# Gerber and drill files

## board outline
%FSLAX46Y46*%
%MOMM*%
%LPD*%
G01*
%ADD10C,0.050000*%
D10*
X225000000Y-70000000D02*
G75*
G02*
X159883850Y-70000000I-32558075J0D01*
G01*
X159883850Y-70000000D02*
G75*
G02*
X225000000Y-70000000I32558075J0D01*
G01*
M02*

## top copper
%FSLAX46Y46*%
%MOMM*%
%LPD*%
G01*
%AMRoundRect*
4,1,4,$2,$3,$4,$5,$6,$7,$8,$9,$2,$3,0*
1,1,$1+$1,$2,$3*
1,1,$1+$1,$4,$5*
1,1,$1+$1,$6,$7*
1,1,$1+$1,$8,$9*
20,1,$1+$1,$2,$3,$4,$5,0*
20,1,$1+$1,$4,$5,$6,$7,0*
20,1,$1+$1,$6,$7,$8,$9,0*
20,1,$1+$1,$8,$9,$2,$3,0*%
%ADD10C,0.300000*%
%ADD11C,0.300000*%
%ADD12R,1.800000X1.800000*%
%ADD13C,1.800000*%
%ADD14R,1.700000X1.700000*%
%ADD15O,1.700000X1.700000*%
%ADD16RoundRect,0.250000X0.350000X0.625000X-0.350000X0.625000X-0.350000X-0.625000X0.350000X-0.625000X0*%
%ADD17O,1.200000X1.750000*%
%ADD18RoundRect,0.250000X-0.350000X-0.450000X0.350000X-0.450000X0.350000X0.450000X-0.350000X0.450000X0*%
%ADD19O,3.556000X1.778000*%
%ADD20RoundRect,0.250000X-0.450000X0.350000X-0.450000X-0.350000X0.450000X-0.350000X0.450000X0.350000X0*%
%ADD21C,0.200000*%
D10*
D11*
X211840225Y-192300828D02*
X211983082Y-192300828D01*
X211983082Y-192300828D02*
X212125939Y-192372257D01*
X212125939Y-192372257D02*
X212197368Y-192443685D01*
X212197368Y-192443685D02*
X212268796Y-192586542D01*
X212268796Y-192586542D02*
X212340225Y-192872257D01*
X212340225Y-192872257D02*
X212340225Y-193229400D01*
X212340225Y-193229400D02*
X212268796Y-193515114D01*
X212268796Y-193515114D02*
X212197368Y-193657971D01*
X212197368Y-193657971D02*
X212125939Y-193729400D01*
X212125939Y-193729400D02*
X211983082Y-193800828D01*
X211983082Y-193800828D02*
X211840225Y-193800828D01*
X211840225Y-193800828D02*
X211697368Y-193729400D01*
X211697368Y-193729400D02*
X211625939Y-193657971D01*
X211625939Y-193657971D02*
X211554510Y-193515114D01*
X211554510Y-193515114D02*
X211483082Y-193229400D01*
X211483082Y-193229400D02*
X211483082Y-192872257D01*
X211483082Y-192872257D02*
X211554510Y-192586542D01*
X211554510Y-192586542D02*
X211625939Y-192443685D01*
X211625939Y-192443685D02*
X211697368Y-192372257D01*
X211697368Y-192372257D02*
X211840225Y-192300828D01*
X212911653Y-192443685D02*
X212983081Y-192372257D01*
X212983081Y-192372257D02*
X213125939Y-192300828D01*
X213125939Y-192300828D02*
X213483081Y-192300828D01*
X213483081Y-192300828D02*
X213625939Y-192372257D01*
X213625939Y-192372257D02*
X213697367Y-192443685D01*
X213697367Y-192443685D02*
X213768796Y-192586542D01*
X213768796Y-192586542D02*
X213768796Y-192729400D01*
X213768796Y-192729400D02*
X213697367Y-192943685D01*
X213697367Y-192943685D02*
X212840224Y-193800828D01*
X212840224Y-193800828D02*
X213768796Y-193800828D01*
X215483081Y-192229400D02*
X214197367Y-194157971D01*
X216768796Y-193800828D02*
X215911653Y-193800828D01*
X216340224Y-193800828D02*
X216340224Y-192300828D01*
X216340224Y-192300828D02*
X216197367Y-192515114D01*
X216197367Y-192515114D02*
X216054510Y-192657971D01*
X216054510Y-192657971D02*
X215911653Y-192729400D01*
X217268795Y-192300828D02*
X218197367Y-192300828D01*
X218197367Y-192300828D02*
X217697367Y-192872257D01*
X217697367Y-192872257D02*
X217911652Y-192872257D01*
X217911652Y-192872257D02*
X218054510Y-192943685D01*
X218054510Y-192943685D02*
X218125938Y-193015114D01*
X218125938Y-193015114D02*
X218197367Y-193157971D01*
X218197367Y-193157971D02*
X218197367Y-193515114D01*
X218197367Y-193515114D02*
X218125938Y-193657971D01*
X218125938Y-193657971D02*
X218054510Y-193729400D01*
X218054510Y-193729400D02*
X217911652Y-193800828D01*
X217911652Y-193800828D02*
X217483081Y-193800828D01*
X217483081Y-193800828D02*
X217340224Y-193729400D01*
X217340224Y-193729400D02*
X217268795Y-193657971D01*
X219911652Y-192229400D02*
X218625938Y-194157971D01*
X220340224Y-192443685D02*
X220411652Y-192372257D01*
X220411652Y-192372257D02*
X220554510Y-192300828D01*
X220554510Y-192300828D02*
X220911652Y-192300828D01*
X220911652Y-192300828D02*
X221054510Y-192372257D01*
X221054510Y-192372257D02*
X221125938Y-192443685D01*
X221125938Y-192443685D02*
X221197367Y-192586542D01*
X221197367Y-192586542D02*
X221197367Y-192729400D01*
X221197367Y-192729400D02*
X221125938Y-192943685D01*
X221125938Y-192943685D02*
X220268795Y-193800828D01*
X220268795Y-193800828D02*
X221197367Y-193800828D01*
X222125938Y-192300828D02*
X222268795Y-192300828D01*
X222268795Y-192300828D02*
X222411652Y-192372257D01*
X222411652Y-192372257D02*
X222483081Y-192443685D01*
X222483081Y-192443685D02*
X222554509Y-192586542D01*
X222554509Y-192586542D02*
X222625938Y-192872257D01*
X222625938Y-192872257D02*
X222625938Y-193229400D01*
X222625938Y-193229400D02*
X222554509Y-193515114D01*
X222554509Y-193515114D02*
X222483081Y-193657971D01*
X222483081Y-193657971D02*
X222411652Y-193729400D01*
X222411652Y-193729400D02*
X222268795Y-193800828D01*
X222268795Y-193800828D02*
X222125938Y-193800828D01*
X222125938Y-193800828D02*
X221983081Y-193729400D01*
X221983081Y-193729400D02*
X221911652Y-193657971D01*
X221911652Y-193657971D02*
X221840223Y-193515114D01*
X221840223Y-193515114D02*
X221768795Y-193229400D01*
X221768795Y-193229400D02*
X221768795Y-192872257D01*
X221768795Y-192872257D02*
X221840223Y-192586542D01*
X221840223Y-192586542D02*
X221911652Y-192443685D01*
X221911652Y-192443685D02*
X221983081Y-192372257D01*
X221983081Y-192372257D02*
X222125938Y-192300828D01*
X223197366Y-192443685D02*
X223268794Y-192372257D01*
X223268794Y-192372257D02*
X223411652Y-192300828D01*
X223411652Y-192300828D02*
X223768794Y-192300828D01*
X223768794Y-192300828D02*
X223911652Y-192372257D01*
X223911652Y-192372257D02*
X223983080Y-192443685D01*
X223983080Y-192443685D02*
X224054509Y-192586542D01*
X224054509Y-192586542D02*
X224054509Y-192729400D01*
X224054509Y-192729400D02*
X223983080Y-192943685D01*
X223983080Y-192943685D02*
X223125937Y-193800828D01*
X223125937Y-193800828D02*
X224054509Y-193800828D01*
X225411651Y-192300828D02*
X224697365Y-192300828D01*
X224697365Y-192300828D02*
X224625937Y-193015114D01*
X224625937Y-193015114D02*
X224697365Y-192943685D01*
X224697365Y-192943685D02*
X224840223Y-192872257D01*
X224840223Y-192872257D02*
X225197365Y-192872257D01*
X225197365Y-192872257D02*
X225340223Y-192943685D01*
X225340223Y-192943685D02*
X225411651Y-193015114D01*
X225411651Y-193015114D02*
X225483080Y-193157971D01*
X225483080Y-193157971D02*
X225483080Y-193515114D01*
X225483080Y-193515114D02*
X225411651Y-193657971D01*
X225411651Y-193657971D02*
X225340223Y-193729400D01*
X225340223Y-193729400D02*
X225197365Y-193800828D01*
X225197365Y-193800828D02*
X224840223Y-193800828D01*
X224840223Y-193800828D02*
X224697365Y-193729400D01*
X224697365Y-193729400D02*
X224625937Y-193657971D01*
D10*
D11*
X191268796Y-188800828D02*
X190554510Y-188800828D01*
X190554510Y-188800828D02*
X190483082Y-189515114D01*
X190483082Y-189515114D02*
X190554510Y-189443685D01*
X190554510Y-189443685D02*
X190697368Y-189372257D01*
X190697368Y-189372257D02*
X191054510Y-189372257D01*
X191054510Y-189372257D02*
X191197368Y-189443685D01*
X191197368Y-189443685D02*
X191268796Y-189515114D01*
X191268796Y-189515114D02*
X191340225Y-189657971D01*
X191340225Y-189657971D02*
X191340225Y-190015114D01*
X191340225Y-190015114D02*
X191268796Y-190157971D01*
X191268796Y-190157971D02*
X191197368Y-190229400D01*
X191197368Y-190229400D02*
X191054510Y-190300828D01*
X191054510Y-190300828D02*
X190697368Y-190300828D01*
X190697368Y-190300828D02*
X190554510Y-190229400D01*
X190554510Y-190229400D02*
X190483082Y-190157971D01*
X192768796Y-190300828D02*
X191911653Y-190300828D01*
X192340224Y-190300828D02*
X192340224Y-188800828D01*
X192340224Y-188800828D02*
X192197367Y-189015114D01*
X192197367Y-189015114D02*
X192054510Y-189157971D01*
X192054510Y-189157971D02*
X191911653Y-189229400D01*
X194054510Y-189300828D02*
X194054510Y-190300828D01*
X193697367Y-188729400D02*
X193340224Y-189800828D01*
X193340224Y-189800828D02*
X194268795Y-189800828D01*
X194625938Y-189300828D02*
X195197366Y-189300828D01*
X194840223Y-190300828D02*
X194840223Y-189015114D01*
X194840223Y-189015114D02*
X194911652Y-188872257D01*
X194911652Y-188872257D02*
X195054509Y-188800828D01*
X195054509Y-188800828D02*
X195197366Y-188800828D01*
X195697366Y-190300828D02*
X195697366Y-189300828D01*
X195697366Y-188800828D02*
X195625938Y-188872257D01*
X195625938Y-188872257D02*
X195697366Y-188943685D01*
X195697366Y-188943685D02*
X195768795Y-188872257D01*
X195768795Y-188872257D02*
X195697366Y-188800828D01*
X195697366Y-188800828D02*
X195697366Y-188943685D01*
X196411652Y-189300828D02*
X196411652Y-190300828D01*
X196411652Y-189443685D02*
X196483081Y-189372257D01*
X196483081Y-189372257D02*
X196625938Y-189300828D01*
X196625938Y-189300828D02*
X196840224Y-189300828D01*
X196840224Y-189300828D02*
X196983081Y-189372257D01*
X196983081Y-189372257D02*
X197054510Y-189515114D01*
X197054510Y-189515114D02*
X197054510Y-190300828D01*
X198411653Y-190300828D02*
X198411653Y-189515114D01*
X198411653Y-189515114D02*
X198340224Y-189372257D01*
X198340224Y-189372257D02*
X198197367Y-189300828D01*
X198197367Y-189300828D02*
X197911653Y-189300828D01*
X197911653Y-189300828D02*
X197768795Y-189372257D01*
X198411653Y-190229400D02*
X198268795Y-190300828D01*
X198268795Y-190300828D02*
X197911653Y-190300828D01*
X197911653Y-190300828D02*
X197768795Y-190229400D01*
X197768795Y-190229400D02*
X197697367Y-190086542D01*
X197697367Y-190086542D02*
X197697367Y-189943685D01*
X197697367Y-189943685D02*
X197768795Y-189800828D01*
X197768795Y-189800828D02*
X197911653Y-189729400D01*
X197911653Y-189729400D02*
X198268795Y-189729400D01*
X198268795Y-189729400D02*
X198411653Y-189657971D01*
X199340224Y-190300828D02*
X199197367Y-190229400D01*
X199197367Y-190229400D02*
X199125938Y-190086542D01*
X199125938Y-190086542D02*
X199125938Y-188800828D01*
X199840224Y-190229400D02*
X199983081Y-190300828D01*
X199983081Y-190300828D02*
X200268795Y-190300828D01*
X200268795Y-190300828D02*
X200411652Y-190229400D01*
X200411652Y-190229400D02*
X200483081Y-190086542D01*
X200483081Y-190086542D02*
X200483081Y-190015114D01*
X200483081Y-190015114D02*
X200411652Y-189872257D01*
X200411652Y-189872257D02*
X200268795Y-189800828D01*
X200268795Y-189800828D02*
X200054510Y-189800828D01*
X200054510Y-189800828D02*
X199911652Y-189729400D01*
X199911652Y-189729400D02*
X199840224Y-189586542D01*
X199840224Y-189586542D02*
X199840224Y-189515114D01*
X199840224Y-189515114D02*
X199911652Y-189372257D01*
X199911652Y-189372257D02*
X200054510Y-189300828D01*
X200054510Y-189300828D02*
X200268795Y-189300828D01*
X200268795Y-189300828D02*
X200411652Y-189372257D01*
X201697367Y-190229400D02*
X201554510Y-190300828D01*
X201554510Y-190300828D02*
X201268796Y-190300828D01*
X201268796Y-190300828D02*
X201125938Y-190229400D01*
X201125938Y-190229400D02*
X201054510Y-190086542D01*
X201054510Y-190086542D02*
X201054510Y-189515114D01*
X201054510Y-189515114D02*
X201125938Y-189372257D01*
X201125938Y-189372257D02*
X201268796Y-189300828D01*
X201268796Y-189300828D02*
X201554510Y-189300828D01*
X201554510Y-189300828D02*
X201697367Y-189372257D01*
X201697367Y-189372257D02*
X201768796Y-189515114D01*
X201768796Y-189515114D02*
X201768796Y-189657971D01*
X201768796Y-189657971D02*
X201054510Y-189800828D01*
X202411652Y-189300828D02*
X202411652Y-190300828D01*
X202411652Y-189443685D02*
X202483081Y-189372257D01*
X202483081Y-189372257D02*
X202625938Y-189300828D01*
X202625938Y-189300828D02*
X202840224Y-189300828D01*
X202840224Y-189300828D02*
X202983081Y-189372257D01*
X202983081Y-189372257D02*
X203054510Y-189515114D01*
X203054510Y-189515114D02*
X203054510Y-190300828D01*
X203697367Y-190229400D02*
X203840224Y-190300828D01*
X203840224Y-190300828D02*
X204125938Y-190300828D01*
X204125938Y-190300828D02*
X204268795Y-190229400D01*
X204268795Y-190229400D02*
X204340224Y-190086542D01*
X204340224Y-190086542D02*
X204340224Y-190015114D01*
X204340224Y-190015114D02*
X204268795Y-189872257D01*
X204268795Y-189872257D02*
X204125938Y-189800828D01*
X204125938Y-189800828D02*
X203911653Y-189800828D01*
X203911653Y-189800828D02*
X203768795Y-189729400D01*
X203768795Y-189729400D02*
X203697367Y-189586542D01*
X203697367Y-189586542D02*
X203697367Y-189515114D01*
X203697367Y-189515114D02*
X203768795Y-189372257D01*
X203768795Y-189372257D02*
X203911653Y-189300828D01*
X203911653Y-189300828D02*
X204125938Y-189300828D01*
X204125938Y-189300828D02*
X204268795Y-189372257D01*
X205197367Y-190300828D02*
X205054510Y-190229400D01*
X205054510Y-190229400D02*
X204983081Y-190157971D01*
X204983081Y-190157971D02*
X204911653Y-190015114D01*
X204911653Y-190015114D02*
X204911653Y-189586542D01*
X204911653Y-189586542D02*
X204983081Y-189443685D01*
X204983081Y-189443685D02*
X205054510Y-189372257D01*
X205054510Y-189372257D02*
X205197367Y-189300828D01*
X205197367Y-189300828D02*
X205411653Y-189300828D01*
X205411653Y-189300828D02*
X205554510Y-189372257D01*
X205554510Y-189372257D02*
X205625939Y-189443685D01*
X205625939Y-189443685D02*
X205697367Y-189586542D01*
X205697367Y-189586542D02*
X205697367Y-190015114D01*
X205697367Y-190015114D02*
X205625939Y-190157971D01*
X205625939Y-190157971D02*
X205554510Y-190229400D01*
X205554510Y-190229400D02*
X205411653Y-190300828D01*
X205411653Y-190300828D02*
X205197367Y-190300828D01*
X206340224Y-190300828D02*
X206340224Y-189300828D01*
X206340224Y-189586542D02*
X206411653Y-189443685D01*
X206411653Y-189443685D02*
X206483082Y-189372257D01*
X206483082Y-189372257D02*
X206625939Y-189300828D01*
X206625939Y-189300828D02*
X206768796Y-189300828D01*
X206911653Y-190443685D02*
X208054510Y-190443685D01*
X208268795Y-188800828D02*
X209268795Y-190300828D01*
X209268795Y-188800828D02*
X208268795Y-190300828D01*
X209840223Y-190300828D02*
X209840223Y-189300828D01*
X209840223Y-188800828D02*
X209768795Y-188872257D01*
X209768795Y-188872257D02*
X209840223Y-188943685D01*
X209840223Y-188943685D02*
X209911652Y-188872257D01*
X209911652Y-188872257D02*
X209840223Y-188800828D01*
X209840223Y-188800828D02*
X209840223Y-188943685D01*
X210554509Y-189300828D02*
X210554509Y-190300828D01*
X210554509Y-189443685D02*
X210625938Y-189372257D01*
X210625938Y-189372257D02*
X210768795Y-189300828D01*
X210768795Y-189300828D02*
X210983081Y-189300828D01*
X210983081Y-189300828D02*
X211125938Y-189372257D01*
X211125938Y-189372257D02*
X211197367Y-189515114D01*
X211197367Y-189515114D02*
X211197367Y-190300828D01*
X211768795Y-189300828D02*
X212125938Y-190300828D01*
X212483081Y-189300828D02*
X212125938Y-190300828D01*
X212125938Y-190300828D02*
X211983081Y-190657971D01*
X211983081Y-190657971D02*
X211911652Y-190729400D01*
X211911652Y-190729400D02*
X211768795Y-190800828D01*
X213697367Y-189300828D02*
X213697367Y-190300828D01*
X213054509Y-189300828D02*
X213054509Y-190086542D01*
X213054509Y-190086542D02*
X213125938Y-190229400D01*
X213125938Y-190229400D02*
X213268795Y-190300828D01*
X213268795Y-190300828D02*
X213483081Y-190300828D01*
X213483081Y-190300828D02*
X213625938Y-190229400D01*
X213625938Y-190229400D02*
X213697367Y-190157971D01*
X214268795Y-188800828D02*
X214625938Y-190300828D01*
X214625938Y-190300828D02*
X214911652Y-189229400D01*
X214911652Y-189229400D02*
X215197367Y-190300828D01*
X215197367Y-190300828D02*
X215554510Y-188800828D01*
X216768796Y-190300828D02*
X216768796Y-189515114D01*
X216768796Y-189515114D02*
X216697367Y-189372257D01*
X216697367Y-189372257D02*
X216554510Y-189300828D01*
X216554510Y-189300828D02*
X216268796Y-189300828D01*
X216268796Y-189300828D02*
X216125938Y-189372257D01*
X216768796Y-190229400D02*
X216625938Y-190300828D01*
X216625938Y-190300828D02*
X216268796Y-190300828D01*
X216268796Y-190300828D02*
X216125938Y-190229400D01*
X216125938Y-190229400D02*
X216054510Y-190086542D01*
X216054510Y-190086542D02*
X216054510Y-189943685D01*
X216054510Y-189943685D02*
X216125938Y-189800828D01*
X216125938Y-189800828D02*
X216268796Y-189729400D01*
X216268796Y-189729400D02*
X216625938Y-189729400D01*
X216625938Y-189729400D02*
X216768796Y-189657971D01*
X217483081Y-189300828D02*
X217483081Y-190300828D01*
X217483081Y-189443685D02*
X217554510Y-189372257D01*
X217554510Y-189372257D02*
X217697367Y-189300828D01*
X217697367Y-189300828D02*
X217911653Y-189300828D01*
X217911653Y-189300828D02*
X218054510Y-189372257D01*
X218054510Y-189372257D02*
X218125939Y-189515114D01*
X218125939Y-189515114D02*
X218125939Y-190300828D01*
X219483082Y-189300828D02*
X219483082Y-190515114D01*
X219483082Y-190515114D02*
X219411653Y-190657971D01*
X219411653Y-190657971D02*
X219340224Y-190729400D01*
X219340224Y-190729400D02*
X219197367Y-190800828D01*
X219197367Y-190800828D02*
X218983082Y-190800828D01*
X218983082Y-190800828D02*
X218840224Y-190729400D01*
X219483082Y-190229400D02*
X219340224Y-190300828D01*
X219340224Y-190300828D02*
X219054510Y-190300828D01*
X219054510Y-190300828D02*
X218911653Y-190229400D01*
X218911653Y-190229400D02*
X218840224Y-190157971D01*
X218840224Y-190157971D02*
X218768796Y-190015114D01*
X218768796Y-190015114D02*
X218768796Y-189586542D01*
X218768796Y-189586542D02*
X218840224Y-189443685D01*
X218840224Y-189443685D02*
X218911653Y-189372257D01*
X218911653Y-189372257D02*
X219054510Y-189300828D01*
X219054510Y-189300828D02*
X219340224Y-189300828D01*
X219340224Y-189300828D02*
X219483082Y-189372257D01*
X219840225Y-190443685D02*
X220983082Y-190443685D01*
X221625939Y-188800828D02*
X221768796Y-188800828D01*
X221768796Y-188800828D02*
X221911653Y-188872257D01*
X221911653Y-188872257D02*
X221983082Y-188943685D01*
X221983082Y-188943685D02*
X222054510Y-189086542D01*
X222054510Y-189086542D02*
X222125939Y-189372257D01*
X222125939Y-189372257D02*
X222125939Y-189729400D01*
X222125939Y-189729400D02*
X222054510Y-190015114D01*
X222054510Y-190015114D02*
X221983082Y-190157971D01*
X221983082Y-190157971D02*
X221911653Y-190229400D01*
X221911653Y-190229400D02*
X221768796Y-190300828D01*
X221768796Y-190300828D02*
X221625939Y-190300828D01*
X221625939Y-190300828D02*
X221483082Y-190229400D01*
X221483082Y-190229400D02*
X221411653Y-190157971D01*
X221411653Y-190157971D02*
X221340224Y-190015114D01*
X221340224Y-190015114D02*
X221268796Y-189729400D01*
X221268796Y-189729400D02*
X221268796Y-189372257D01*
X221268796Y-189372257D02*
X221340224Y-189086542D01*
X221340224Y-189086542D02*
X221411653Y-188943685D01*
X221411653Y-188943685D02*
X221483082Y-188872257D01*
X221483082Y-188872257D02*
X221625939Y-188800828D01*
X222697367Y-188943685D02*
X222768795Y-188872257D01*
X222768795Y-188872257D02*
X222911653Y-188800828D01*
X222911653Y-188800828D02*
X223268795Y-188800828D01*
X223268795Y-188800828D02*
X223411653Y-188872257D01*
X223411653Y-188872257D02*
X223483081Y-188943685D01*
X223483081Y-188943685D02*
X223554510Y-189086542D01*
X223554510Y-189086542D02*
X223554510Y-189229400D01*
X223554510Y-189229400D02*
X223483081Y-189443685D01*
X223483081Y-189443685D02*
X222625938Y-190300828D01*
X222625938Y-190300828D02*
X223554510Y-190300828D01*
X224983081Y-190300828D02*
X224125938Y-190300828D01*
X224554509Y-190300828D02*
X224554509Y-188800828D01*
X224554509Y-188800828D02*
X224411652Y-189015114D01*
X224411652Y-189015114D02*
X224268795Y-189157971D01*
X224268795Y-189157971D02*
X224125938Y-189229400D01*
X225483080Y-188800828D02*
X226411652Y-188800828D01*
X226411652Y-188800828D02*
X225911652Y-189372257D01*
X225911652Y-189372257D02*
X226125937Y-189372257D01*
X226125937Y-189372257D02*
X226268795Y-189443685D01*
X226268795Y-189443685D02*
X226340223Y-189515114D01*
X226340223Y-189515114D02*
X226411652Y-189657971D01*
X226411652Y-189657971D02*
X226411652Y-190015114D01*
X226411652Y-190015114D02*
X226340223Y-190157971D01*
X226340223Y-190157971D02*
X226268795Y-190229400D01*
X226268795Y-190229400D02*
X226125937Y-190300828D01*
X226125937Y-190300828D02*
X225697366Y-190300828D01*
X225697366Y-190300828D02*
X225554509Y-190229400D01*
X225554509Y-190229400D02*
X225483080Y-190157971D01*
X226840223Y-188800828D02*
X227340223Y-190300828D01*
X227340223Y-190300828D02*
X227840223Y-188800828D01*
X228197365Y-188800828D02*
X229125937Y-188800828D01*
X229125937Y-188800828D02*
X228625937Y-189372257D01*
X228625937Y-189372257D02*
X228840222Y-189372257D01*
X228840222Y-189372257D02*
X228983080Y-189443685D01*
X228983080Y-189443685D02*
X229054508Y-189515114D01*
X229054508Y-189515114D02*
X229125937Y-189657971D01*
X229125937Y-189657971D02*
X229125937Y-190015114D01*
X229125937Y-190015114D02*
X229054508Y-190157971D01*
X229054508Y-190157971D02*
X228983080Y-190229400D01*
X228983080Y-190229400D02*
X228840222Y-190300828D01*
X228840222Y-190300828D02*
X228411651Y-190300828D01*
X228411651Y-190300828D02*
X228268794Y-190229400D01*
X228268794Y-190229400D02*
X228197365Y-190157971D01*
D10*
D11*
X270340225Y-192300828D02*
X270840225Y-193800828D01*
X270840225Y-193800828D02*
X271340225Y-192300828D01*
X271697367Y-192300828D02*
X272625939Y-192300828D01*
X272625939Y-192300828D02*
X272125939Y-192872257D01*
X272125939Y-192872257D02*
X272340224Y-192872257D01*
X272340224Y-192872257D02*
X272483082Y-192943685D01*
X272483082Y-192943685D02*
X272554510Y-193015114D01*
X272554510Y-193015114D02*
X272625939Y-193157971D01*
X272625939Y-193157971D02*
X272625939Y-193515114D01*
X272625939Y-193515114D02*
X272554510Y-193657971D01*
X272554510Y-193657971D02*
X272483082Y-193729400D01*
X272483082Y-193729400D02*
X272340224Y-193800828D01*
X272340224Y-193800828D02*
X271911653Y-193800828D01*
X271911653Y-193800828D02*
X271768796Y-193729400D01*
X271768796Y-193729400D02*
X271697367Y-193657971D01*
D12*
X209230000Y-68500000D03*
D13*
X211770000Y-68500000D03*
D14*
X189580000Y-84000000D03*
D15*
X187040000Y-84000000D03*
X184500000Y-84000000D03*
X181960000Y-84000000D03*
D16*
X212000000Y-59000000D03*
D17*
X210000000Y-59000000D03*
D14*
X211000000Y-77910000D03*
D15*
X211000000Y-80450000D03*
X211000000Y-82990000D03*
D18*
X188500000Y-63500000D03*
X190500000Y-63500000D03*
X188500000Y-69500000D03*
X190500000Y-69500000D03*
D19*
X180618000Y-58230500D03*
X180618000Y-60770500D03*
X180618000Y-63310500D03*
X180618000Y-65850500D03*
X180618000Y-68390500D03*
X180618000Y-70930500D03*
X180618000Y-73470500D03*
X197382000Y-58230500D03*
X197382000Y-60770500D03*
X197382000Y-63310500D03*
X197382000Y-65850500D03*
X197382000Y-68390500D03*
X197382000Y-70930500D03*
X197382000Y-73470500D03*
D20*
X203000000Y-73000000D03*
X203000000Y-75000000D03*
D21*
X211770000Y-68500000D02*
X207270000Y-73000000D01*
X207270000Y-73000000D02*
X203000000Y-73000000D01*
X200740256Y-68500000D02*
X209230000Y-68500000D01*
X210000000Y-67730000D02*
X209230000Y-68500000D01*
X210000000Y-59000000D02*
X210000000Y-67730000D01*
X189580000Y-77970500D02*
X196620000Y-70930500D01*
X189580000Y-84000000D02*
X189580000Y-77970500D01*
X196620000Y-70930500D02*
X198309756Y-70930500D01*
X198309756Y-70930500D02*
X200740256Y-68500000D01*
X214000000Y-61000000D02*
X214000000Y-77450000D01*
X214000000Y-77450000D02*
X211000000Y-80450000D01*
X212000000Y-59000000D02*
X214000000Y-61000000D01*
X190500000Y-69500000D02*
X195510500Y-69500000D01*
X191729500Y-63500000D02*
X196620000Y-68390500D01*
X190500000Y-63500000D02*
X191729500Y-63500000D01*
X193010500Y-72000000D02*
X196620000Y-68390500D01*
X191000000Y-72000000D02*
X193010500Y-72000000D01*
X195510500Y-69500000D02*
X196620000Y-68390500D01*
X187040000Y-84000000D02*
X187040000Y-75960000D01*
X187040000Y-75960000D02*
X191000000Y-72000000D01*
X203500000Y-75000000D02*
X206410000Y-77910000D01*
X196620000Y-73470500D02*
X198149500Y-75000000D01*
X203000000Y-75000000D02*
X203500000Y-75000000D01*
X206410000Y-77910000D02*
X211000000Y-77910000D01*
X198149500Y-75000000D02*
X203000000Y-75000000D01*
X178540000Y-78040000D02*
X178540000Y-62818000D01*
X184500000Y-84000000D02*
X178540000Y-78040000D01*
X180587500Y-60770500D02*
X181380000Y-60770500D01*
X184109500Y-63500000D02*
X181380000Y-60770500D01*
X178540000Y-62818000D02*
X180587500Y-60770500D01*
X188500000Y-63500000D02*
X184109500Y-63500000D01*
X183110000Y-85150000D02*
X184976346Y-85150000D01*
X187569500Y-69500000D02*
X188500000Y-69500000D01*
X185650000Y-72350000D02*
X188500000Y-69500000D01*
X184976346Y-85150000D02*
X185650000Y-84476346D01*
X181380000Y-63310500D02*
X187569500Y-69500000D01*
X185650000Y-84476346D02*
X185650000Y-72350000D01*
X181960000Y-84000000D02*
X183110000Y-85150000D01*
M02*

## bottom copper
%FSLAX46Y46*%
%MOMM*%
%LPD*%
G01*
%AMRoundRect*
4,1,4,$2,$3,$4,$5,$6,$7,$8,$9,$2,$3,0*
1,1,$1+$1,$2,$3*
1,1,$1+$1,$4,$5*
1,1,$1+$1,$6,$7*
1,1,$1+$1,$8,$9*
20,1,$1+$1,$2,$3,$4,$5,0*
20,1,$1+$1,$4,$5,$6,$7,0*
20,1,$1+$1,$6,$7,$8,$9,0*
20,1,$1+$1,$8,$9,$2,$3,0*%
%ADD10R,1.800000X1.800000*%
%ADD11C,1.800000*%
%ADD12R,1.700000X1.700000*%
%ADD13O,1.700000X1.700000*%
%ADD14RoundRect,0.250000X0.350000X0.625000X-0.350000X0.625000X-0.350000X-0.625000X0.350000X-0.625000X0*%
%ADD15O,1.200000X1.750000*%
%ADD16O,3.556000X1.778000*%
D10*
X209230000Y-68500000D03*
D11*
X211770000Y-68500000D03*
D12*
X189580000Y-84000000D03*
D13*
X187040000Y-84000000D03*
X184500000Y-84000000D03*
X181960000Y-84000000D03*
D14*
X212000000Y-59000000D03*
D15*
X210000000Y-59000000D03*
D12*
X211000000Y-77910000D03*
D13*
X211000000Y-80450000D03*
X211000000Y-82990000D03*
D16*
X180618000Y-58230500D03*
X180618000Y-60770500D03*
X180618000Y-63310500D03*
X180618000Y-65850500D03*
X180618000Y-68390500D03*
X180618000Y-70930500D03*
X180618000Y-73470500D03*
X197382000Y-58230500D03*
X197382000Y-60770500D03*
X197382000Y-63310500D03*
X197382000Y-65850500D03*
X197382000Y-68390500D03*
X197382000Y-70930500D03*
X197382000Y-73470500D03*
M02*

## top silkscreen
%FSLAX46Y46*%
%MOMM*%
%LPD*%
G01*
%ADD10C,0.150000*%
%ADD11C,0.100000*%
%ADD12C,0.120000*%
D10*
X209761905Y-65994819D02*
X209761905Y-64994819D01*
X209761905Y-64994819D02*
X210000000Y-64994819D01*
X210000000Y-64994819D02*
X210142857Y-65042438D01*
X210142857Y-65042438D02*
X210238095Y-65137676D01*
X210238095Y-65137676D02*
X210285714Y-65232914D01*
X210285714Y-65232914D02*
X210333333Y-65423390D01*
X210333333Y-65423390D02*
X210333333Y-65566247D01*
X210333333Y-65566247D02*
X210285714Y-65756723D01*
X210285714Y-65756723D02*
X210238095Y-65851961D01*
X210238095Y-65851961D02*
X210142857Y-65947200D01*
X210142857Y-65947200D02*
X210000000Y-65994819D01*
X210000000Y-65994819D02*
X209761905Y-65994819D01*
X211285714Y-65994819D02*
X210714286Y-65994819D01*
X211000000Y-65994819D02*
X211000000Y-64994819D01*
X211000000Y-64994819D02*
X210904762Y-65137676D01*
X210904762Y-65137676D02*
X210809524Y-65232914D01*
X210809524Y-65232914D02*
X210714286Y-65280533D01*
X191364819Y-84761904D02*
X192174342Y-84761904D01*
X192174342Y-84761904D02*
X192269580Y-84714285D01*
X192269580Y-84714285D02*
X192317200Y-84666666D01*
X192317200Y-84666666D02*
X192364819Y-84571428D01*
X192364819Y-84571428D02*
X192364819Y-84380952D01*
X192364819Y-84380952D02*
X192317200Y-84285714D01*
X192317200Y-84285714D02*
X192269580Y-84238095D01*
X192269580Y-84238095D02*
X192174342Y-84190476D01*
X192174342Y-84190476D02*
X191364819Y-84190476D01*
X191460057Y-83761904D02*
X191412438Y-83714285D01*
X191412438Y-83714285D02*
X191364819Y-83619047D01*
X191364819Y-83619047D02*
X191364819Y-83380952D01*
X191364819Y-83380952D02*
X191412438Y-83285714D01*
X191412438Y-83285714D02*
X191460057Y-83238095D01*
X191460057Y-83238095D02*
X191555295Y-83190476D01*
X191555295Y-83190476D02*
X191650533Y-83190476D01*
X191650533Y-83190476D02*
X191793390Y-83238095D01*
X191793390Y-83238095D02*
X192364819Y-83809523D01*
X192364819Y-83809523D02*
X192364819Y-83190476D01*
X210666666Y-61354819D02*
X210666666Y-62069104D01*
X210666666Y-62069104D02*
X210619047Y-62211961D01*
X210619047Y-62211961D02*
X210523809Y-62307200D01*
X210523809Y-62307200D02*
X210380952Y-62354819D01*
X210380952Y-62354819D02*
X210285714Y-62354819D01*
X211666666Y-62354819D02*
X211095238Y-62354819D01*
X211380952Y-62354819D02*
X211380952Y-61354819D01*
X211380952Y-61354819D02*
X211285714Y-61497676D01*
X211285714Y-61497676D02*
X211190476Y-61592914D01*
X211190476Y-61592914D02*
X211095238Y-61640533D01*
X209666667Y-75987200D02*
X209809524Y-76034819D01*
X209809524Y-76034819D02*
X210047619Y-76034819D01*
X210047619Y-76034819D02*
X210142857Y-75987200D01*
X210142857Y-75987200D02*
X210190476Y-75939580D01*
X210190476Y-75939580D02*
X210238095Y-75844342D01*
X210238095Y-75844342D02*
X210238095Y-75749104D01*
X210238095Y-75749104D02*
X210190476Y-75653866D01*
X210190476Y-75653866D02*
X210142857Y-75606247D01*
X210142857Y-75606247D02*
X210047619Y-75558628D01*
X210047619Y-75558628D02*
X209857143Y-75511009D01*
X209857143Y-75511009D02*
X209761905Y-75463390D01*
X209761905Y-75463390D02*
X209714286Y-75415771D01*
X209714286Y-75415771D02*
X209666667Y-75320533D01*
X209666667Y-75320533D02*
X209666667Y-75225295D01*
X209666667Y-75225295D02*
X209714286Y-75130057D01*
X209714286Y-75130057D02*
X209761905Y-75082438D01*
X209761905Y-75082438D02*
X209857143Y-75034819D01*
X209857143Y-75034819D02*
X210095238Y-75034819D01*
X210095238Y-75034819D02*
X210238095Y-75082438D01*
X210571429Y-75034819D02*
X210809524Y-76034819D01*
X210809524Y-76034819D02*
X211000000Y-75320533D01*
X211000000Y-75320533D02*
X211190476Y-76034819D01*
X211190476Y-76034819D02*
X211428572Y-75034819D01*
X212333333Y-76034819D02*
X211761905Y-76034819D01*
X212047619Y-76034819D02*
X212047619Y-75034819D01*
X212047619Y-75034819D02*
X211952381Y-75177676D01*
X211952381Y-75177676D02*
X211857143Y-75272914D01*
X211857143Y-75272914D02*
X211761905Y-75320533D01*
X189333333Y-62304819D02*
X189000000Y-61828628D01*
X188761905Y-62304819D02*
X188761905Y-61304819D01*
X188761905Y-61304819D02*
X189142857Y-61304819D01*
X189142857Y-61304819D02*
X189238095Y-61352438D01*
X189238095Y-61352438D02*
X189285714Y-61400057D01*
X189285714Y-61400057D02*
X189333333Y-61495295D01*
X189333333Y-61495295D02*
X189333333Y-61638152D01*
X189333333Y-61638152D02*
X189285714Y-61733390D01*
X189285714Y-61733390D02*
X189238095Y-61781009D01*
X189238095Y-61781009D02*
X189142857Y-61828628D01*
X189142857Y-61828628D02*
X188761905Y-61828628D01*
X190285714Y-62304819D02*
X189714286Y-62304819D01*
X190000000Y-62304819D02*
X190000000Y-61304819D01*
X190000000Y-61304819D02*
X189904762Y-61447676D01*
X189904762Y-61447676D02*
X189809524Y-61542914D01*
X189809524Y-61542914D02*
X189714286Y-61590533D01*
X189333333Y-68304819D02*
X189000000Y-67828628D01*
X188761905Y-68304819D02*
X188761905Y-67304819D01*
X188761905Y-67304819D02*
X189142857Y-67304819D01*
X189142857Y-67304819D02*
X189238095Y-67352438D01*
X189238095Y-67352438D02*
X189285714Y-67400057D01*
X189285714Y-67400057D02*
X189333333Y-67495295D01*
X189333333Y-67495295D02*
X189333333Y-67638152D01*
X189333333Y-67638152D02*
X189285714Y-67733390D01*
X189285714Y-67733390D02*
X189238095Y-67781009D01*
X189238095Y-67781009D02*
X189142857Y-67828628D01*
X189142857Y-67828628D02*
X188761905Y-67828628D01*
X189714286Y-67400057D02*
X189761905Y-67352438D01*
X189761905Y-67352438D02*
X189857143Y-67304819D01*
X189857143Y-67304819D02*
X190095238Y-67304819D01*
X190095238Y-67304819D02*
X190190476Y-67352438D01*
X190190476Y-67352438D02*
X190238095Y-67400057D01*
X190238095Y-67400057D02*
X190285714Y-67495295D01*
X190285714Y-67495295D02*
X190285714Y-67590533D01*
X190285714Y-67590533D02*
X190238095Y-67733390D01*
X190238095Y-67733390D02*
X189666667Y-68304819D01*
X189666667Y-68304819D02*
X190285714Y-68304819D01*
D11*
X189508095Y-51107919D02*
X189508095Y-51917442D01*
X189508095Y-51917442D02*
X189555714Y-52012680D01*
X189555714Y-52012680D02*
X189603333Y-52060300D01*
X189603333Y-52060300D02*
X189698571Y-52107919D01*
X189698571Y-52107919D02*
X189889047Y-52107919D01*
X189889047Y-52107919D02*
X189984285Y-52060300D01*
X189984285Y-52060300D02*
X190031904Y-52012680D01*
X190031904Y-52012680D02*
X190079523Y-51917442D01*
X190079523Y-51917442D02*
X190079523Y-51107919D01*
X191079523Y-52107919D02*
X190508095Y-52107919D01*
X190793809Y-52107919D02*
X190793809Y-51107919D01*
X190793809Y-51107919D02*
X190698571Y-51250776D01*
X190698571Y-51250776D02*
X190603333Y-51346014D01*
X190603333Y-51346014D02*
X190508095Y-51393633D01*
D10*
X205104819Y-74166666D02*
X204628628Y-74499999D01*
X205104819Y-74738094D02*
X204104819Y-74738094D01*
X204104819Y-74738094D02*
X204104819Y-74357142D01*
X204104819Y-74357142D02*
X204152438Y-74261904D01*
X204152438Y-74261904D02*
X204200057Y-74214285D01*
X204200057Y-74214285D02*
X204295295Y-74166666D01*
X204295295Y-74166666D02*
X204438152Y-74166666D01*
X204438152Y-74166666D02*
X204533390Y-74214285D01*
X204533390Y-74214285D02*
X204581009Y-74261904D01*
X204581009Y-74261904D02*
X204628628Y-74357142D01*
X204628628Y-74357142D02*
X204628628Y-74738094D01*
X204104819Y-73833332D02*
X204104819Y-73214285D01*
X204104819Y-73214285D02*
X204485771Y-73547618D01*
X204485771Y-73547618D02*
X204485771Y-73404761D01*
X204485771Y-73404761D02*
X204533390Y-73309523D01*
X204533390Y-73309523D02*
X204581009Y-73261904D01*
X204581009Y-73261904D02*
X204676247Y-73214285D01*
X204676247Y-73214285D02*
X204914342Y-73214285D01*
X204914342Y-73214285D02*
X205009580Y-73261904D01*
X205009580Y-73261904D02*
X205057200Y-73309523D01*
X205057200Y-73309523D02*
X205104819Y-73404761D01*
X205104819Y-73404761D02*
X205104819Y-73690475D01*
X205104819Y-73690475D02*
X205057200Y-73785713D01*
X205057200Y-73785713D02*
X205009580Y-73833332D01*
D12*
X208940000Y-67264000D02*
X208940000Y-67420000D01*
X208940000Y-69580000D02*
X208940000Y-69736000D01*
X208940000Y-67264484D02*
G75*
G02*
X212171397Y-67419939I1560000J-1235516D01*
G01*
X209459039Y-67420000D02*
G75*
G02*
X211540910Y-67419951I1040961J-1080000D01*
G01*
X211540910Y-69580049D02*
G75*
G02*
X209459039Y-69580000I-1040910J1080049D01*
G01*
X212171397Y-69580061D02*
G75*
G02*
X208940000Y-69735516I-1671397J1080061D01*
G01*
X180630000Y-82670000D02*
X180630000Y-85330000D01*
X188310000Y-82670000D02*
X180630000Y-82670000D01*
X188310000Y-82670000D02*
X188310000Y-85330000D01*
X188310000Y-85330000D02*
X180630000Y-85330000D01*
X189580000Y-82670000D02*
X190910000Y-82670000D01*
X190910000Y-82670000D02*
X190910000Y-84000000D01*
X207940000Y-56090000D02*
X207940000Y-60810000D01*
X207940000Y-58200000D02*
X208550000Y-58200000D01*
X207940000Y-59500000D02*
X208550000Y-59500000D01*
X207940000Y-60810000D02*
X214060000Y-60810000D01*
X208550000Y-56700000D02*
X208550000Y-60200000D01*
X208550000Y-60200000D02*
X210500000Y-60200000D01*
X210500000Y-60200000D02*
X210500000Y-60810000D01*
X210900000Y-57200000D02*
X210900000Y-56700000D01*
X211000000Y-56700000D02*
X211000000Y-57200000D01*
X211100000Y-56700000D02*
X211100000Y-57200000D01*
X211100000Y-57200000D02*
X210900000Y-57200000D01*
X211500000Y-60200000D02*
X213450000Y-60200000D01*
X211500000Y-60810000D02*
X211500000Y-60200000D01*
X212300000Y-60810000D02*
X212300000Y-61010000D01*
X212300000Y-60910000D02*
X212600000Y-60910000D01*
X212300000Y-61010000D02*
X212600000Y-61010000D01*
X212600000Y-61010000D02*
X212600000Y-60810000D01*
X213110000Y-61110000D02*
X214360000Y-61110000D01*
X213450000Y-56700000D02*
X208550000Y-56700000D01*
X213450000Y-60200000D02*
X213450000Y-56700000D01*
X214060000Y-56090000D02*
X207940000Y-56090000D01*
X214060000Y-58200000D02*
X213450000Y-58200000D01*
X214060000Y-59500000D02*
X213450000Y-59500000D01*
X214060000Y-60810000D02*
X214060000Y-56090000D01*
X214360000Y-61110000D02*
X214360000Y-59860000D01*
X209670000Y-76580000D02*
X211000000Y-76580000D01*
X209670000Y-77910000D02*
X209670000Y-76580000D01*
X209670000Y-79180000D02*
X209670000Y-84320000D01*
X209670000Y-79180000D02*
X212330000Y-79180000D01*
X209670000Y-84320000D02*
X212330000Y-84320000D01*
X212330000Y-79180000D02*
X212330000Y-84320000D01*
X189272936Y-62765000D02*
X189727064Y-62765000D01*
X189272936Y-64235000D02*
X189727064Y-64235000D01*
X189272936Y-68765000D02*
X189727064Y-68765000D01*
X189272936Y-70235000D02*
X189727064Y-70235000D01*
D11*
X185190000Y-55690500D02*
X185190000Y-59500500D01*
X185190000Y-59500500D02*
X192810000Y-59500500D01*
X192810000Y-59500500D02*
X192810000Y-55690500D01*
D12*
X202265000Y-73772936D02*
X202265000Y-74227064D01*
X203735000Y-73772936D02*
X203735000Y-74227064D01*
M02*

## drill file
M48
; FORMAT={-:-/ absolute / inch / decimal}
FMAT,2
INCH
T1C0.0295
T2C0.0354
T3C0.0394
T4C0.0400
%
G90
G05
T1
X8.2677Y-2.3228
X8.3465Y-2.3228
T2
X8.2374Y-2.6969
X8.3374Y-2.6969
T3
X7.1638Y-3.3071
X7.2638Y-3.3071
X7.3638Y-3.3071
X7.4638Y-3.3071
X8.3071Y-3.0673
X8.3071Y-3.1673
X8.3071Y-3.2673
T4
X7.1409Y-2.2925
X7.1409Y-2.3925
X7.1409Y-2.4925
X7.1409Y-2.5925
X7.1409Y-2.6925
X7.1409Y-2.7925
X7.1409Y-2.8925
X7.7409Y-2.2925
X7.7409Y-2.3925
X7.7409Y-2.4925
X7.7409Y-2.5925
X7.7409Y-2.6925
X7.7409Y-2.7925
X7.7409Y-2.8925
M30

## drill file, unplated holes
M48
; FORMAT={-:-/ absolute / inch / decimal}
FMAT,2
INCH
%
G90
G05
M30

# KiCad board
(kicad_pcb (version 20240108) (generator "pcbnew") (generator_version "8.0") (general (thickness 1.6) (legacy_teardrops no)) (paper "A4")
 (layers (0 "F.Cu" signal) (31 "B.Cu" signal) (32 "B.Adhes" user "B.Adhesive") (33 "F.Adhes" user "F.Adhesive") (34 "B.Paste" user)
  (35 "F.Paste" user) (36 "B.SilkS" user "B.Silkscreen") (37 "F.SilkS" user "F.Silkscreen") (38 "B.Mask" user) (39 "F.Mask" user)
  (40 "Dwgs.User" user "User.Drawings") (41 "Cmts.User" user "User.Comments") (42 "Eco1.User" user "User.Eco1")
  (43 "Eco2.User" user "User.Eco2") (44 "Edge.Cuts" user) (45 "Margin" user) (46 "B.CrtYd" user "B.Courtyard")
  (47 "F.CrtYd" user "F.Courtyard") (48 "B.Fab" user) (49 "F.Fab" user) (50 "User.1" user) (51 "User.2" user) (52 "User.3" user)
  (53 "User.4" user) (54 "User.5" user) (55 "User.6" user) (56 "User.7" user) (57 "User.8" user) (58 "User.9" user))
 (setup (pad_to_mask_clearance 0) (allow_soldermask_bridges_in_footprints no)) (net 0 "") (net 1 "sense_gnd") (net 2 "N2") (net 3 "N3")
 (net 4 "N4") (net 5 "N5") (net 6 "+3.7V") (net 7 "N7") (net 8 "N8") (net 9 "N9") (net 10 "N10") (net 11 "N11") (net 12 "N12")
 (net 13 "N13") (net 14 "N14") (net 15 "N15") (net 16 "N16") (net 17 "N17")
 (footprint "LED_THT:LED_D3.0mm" (layer "F.Cu") (at 209.23 68.5)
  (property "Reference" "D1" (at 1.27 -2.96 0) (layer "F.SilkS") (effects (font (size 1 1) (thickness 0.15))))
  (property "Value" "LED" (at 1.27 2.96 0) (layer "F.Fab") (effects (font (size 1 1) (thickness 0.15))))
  (fp_line (start -0.29 -1.236) (end -0.29 -1.08) (stroke (width 0.12) (type solid)) (layer "F.SilkS"))
  (fp_line (start -0.29 1.08) (end -0.29 1.236) (stroke (width 0.12) (type solid)) (layer "F.SilkS"))
  (fp_arc (start -0.29 -1.235516) (mid 1.365624 -1.987701) (end 2.941397 -1.080061) (stroke (width 0.12) (type solid)) (layer "F.SilkS"))
  (fp_arc (start 0.229039 -1.08) (mid 1.269965 -1.5) (end 2.31091 -1.080049) (stroke (width 0.12) (type solid)) (layer "F.SilkS"))
  (fp_arc (start 2.31091 1.080049) (mid 1.269965 1.5) (end 0.229039 1.08) (stroke (width 0.12) (type solid)) (layer "F.SilkS"))
  (fp_arc (start 2.941397 1.080061) (mid 1.365624 1.987701) (end -0.29 1.235516) (stroke (width 0.12) (type solid)) (layer "F.SilkS"))
  (pad "1" thru_hole rect (at 0 0) (size 1.8 1.8) (drill 0.9) (layers "*.Cu" "*.Mask") (remove_unused_layers no) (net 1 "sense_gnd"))
  (pad "2" thru_hole circle (at 2.54 0) (size 1.8 1.8) (drill 0.9) (layers "*.Cu" "*.Mask") (remove_unused_layers no) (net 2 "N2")))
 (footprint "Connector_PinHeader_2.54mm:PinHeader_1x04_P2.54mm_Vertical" (layer "F.Cu") (at 189.58 84 -90)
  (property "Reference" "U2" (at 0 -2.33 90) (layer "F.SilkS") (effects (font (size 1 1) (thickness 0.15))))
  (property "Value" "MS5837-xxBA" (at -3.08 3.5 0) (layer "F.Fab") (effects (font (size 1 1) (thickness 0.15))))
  (fp_line (start -1.33 8.95) (end 1.33 8.95) (stroke (width 0.12) (type solid)) (layer "F.SilkS"))
  (fp_line (start -1.33 1.27) (end -1.33 8.95) (stroke (width 0.12) (type solid)) (layer "F.SilkS"))
  (fp_line (start -1.33 1.27) (end 1.33 1.27) (stroke (width 0.12) (type solid)) (layer "F.SilkS"))
  (fp_line (start 1.33 1.27) (end 1.33 8.95) (stroke (width 0.12) (type solid)) (layer "F.SilkS"))
  (fp_line (start -1.33 0) (end -1.33 -1.33) (stroke (width 0.12) (type solid)) (layer "F.SilkS"))
  (fp_line (start -1.33 -1.33) (end 0 -1.33) (stroke (width 0.12) (type solid)) (layer "F.SilkS"))
  (pad "1" thru_hole rect (at 0 0 270) (size 1.7 1.7) (drill 1) (layers "*.Cu" "*.Mask") (remove_unused_layers no) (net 1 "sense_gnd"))
  (pad "2" thru_hole oval (at 0 2.54 270) (size 1.7 1.7) (drill 1) (layers "*.Cu" "*.Mask") (remove_unused_layers no) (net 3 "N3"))
  (pad "3" thru_hole oval (at 0 5.08 270) (size 1.7 1.7) (drill 1) (layers "*.Cu" "*.Mask") (remove_unused_layers no) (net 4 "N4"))
  (pad "4" thru_hole oval (at 0 7.62 270) (size 1.7 1.7) (drill 1) (layers "*.Cu" "*.Mask") (remove_unused_layers no) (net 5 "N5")))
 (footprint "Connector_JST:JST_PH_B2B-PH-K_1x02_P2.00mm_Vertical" (layer "F.Cu") (at 212 59 180)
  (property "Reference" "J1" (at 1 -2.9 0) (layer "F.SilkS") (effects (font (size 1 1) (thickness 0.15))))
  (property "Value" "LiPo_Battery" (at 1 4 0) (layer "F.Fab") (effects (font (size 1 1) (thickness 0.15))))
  (fp_line (start 4.06 2.91) (end 4.06 -1.81) (stroke (width 0.12) (type solid)) (layer "F.SilkS"))
  (fp_line (start 4.06 0.8) (end 3.45 0.8) (stroke (width 0.12) (type solid)) (layer "F.SilkS"))
  (fp_line (start 4.06 -0.5) (end 3.45 -0.5) (stroke (width 0.12) (type solid)) (layer "F.SilkS"))
  (fp_line (start 4.06 -1.81) (end -2.06 -1.81) (stroke (width 0.12) (type solid)) (layer "F.SilkS"))
  (fp_line (start 3.45 2.3) (end 3.45 -1.2) (stroke (width 0.12) (type solid)) (layer "F.SilkS"))
  (fp_line (start 3.45 -1.2) (end 1.5 -1.2) (stroke (width 0.12) (type solid)) (layer "F.SilkS"))
  (fp_line (start 1.5 -1.2) (end 1.5 -1.81) (stroke (width 0.12) (type solid)) (layer "F.SilkS"))
  (fp_line (start 1.1 1.8) (end 1.1 2.3) (stroke (width 0.12) (type solid)) (layer "F.SilkS"))
  (fp_line (start 1 2.3) (end 1 1.8) (stroke (width 0.12) (type solid)) (layer "F.SilkS"))
  (fp_line (start 0.9 2.3) (end 0.9 1.8) (stroke (width 0.12) (type solid)) (layer "F.SilkS"))
  (fp_line (start 0.9 1.8) (end 1.1 1.8) (stroke (width 0.12) (type solid)) (layer "F.SilkS"))
  (fp_line (start 0.5 -1.2) (end -1.45 -1.2) (stroke (width 0.12) (type solid)) (layer "F.SilkS"))
  (fp_line (start 0.5 -1.81) (end 0.5 -1.2) (stroke (width 0.12) (type solid)) (layer "F.SilkS"))
  (fp_line (start -0.3 -1.81) (end -0.3 -2.01) (stroke (width 0.12) (type solid)) (layer "F.SilkS"))
  (fp_line (start -0.3 -1.91) (end -0.6 -1.91) (stroke (width 0.12) (type solid)) (layer "F.SilkS"))
  (fp_line (start -0.3 -2.01) (end -0.6 -2.01) (stroke (width 0.12) (type solid)) (layer "F.SilkS"))
  (fp_line (start -0.6 -2.01) (end -0.6 -1.81) (stroke (width 0.12) (type solid)) (layer "F.SilkS"))
  (fp_line (start -1.11 -2.11) (end -2.36 -2.11) (stroke (width 0.12) (type solid)) (layer "F.SilkS"))
  (fp_line (start -1.45 2.3) (end 3.45 2.3) (stroke (width 0.12) (type solid)) (layer "F.SilkS"))
  (fp_line (start -1.45 -1.2) (end -1.45 2.3) (stroke (width 0.12) (type solid)) (layer "F.SilkS"))
  (fp_line (start -2.06 2.91) (end 4.06 2.91) (stroke (width 0.12) (type solid)) (layer "F.SilkS"))
  (fp_line (start -2.06 0.8) (end -1.45 0.8) (stroke (width 0.12) (type solid)) (layer "F.SilkS"))
  (fp_line (start -2.06 -0.5) (end -1.45 -0.5) (stroke (width 0.12) (type solid)) (layer "F.SilkS"))
  (fp_line (start -2.06 -1.81) (end -2.06 2.91) (stroke (width 0.12) (type solid)) (layer "F.SilkS"))
  (fp_line (start -2.36 -2.11) (end -2.36 -0.86) (stroke (width 0.12) (type solid)) (layer "F.SilkS"))
  (pad "1" thru_hole roundrect (at 0 0 180) (size 1.2 1.75) (drill 0.75) (layers "*.Cu" "*.Mask") (remove_unused_layers no)
   (roundrect_rratio 0.208333) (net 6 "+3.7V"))
  (pad "2" thru_hole oval (at 2 0 180) (size 1.2 1.75) (drill 0.75) (layers "*.Cu" "*.Mask") (remove_unused_layers no) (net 1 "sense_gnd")))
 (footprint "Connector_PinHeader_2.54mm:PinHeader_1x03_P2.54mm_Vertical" (layer "F.Cu") (at 211 77.91)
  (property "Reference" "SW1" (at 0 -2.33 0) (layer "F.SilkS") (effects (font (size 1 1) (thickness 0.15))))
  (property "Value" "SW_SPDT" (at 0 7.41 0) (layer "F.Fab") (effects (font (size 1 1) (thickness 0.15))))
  (fp_line (start -1.33 -1.33) (end 0 -1.33) (stroke (width 0.12) (type solid)) (layer "F.SilkS"))
  (fp_line (start -1.33 0) (end -1.33 -1.33) (stroke (width 0.12) (type solid)) (layer "F.SilkS"))
  (fp_line (start -1.33 1.27) (end -1.33 6.41) (stroke (width 0.12) (type solid)) (layer "F.SilkS"))
  (fp_line (start -1.33 1.27) (end 1.33 1.27) (stroke (width 0.12) (type solid)) (layer "F.SilkS"))
  (fp_line (start -1.33 6.41) (end 1.33 6.41) (stroke (width 0.12) (type solid)) (layer "F.SilkS"))
  (fp_line (start 1.33 1.27) (end 1.33 6.41) (stroke (width 0.12) (type solid)) (layer "F.SilkS"))
  (pad "1" thru_hole rect (at 0 0) (size 1.7 1.7) (drill 1) (layers "*.Cu" "*.Mask") (remove_unused_layers no) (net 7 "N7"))
  (pad "2" thru_hole oval (at 0 2.54) (size 1.7 1.7) (drill 1) (layers "*.Cu" "*.Mask") (remove_unused_layers no) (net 6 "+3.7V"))
  (pad "3" thru_hole oval (at 0 5.08) (size 1.7 1.7) (drill 1) (layers "*.Cu" "*.Mask") (remove_unused_layers no) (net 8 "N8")))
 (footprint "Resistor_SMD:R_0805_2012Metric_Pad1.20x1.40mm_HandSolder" (layer "F.Cu") (at 189.5 63.5)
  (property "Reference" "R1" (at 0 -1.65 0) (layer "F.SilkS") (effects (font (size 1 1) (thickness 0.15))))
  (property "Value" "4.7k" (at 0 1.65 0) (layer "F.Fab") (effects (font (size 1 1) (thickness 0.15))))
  (fp_line (start -0.227064 -0.735) (end 0.227064 -0.735) (stroke (width 0.12) (type solid)) (layer "F.SilkS"))
  (fp_line (start -0.227064 0.735) (end 0.227064 0.735) (stroke (width 0.12) (type solid)) (layer "F.SilkS"))
  (pad "1" smd roundrect (at -1 0) (size 1.2 1.4) (layers "F.Cu" "F.Paste" "F.Mask") (roundrect_rratio 0.208333) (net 4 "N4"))
  (pad "2" smd roundrect (at 1 0) (size 1.2 1.4) (layers "F.Cu" "F.Paste" "F.Mask") (roundrect_rratio 0.208333) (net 3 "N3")))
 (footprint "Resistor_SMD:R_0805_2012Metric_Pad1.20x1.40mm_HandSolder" (layer "F.Cu") (at 189.5 69.5)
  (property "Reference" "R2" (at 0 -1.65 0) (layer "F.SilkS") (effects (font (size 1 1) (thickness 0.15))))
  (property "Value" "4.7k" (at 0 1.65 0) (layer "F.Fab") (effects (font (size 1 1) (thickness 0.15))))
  (fp_line (start -0.227064 -0.735) (end 0.227064 -0.735) (stroke (width 0.12) (type solid)) (layer "F.SilkS"))
  (fp_line (start -0.227064 0.735) (end 0.227064 0.735) (stroke (width 0.12) (type solid)) (layer "F.SilkS"))
  (pad "1" smd roundrect (at -1 0) (size 1.2 1.4) (layers "F.Cu" "F.Paste" "F.Mask") (roundrect_rratio 0.208333) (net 5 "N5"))
  (pad "2" smd roundrect (at 1 0) (size 1.2 1.4) (layers "F.Cu" "F.Paste" "F.Mask") (roundrect_rratio 0.208333) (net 3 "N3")))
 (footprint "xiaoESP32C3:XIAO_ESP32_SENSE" (layer "F.Cu") (at 189 65.8505)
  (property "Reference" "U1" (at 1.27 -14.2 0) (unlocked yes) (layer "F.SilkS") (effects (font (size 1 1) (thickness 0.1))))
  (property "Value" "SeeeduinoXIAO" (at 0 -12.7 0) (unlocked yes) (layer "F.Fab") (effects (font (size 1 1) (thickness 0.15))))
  (fp_line (start -3.81 -10.16) (end -3.81 -6.35) (stroke (width 0.1) (type default)) (layer "F.SilkS"))
  (fp_line (start -3.81 -6.35) (end 3.81 -6.35) (stroke (width 0.1) (type default)) (layer "F.SilkS"))
  (fp_line (start 3.81 -6.35) (end 3.81 -10.16) (stroke (width 0.1) (type default)) (layer "F.SilkS"))
  (pad "1" thru_hole oval (at -7.62 -7.62) (size 3.556 1.778) (drill 1.016 (offset -0.762 0)) (layers "*.Cu" "*.Mask")
   (remove_unused_layers no) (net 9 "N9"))
  (pad "2" thru_hole oval (at -7.62 -5.08) (size 3.556 1.778) (drill 1.016 (offset -0.762 0)) (layers "*.Cu" "*.Mask")
   (remove_unused_layers no) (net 4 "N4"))
  (pad "3" thru_hole oval (at -7.62 -2.54) (size 3.556 1.778) (drill 1.016 (offset -0.762 0)) (layers "*.Cu" "*.Mask")
   (remove_unused_layers no) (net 5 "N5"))
  (pad "4" thru_hole oval (at -7.62 0) (size 3.556 1.778) (drill 1.016 (offset -0.762 0)) (layers "*.Cu" "*.Mask") (remove_unused_layers no)
   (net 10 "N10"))
  (pad "5" thru_hole oval (at -7.62 2.54) (size 3.556 1.778) (drill 1.016 (offset -0.762 0)) (layers "*.Cu" "*.Mask")
   (remove_unused_layers no) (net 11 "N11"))
  (pad "6" thru_hole oval (at -7.62 5.08) (size 3.556 1.778) (drill 1.016 (offset -0.762 0)) (layers "*.Cu" "*.Mask")
   (remove_unused_layers no) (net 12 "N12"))
  (pad "7" thru_hole oval (at -7.62 7.62) (size 3.556 1.778) (drill 1.016 (offset -0.762 0)) (layers "*.Cu" "*.Mask")
   (remove_unused_layers no) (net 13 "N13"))
  (pad "8" thru_hole oval (at 7.62 -7.62) (size 3.556 1.778) (drill 1.016 (offset 0.762 0)) (layers "*.Cu" "*.Mask")
   (remove_unused_layers no) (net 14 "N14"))
  (pad "9" thru_hole oval (at 7.62 -5.08) (size 3.556 1.778) (drill 1.016 (offset 0.762 0)) (layers "*.Cu" "*.Mask")
   (remove_unused_layers no) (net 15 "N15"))
  (pad "10" thru_hole oval (at 7.62 -2.54) (size 3.556 1.778) (drill 1.016 (offset 0.762 0)) (layers "*.Cu" "*.Mask")
   (remove_unused_layers no) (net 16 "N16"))
  (pad "11" thru_hole oval (at 7.62 0) (size 3.556 1.778) (drill 1.016 (offset 0.762 0)) (layers "*.Cu" "*.Mask") (remove_unused_layers no)
   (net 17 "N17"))
  (pad "12" thru_hole oval (at 7.62 2.54) (size 3.556 1.778) (drill 1.016 (offset 0.762 0)) (layers "*.Cu" "*.Mask")
   (remove_unused_layers no) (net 3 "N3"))
  (pad "13" thru_hole oval (at 7.62 5.08) (size 3.556 1.778) (drill 1.016 (offset 0.762 0)) (layers "*.Cu" "*.Mask")
   (remove_unused_layers no) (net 1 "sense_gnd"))
  (pad "14" thru_hole oval (at 7.62 7.62) (size 3.556 1.778) (drill 1.016 (offset 0.762 0)) (layers "*.Cu" "*.Mask")
   (remove_unused_layers no) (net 7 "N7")))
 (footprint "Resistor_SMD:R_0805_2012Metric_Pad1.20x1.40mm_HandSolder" (layer "F.Cu") (at 203 74 -90)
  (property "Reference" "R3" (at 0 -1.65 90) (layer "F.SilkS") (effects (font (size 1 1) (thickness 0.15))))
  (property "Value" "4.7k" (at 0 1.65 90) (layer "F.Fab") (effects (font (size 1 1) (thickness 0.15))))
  (fp_line (start -0.227064 0.735) (end 0.227064 0.735) (stroke (width 0.12) (type solid)) (layer "F.SilkS"))
  (fp_line (start -0.227064 -0.735) (end 0.227064 -0.735) (stroke (width 0.12) (type solid)) (layer "F.SilkS"))
  (pad "1" smd roundrect (at -1 0 270) (size 1.2 1.4) (layers "F.Cu" "F.Paste" "F.Mask") (roundrect_rratio 0.208333) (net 2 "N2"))
  (pad "2" smd roundrect (at 1 0 270) (size 1.2 1.4) (layers "F.Cu" "F.Paste" "F.Mask") (roundrect_rratio 0.208333) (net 7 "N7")))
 (gr_circle (center 192.441925 70) (end 220.509313 86.5) (stroke (width 0.05) (type default)) (fill none) (layer "Edge.Cuts"))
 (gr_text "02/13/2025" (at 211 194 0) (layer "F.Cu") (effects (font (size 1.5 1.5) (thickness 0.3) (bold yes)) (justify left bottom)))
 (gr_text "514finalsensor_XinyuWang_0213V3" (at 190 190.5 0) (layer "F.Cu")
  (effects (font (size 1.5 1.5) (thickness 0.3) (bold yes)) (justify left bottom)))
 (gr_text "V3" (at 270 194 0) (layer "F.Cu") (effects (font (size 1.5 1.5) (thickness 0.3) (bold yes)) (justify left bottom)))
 (segment (start 211.77 68.5) (end 207.27 73) (width 0.2) (layer "F.Cu") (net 2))
 (segment (start 207.27 73) (end 203 73) (width 0.2) (layer "F.Cu") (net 2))
 (segment (start 200.740256 68.5) (end 209.23 68.5) (width 0.2) (layer "F.Cu") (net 1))
 (segment (start 210 67.73) (end 209.23 68.5) (width 0.2) (layer "F.Cu") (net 1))
 (segment (start 210 59) (end 210 67.73) (width 0.2) (layer "F.Cu") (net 1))
 (segment (start 189.58 77.9705) (end 196.62 70.9305) (width 0.2) (layer "F.Cu") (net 1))
 (segment (start 189.58 84) (end 189.58 77.9705) (width 0.2) (layer "F.Cu") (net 1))
 (segment (start 196.62 70.9305) (end 198.309756 70.9305) (width 0.2) (layer "F.Cu") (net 1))
 (segment (start 198.309756 70.9305) (end 200.740256 68.5) (width 0.2) (layer "F.Cu") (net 1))
 (segment (start 214 61) (end 214 77.45) (width 0.2) (layer "F.Cu") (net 6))
 (segment (start 214 77.45) (end 211 80.45) (width 0.2) (layer "F.Cu") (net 6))
 (segment (start 212 59) (end 214 61) (width 0.2) (layer "F.Cu") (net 6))
 (segment (start 190.5 69.5) (end 195.5105 69.5) (width 0.2) (layer "F.Cu") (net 3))
 (segment (start 191.7295 63.5) (end 196.62 68.3905) (width 0.2) (layer "F.Cu") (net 3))
 (segment (start 190.5 63.5) (end 191.7295 63.5) (width 0.2) (layer "F.Cu") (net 3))
 (segment (start 193.0105 72) (end 196.62 68.3905) (width 0.2) (layer "F.Cu") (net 3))
 (segment (start 191 72) (end 193.0105 72) (width 0.2) (layer "F.Cu") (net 3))
 (segment (start 195.5105 69.5) (end 196.62 68.3905) (width 0.2) (layer "F.Cu") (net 3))
 (segment (start 187.04 84) (end 187.04 75.96) (width 0.2) (layer "F.Cu") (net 3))
 (segment (start 187.04 75.96) (end 191 72) (width 0.2) (layer "F.Cu") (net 3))
 (segment (start 203.5 75) (end 206.41 77.91) (width 0.2) (layer "F.Cu") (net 7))
 (segment (start 196.62 73.4705) (end 198.1495 75) (width 0.2) (layer "F.Cu") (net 7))
 (segment (start 203 75) (end 203.5 75) (width 0.2) (layer "F.Cu") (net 7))
 (segment (start 206.41 77.91) (end 211 77.91) (width 0.2) (layer "F.Cu") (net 7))
 (segment (start 198.1495 75) (end 203 75) (width 0.2) (layer "F.Cu") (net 7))
 (segment (start 178.54 78.04) (end 178.54 62.818) (width 0.2) (layer "F.Cu") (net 4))
 (segment (start 184.5 84) (end 178.54 78.04) (width 0.2) (layer "F.Cu") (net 4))
 (segment (start 180.5875 60.7705) (end 181.38 60.7705) (width 0.2) (layer "F.Cu") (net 4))
 (segment (start 184.1095 63.5) (end 181.38 60.7705) (width 0.2) (layer "F.Cu") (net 4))
 (segment (start 178.54 62.818) (end 180.5875 60.7705) (width 0.2) (layer "F.Cu") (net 4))
 (segment (start 188.5 63.5) (end 184.1095 63.5) (width 0.2) (layer "F.Cu") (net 4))
 (segment (start 183.11 85.15) (end 184.976346 85.15) (width 0.2) (layer "F.Cu") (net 5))
 (segment (start 187.5695 69.5) (end 188.5 69.5) (width 0.2) (layer "F.Cu") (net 5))
 (segment (start 185.65 72.35) (end 188.5 69.5) (width 0.2) (layer "F.Cu") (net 5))
 (segment (start 184.976346 85.15) (end 185.65 84.476346) (width 0.2) (layer "F.Cu") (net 5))
 (segment (start 181.38 63.3105) (end 187.5695 69.5) (width 0.2) (layer "F.Cu") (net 5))
 (segment (start 185.65 84.476346) (end 185.65 72.35) (width 0.2) (layer "F.Cu") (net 5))
 (segment (start 181.96 84) (end 183.11 85.15) (width 0.2) (layer "F.Cu") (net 5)))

